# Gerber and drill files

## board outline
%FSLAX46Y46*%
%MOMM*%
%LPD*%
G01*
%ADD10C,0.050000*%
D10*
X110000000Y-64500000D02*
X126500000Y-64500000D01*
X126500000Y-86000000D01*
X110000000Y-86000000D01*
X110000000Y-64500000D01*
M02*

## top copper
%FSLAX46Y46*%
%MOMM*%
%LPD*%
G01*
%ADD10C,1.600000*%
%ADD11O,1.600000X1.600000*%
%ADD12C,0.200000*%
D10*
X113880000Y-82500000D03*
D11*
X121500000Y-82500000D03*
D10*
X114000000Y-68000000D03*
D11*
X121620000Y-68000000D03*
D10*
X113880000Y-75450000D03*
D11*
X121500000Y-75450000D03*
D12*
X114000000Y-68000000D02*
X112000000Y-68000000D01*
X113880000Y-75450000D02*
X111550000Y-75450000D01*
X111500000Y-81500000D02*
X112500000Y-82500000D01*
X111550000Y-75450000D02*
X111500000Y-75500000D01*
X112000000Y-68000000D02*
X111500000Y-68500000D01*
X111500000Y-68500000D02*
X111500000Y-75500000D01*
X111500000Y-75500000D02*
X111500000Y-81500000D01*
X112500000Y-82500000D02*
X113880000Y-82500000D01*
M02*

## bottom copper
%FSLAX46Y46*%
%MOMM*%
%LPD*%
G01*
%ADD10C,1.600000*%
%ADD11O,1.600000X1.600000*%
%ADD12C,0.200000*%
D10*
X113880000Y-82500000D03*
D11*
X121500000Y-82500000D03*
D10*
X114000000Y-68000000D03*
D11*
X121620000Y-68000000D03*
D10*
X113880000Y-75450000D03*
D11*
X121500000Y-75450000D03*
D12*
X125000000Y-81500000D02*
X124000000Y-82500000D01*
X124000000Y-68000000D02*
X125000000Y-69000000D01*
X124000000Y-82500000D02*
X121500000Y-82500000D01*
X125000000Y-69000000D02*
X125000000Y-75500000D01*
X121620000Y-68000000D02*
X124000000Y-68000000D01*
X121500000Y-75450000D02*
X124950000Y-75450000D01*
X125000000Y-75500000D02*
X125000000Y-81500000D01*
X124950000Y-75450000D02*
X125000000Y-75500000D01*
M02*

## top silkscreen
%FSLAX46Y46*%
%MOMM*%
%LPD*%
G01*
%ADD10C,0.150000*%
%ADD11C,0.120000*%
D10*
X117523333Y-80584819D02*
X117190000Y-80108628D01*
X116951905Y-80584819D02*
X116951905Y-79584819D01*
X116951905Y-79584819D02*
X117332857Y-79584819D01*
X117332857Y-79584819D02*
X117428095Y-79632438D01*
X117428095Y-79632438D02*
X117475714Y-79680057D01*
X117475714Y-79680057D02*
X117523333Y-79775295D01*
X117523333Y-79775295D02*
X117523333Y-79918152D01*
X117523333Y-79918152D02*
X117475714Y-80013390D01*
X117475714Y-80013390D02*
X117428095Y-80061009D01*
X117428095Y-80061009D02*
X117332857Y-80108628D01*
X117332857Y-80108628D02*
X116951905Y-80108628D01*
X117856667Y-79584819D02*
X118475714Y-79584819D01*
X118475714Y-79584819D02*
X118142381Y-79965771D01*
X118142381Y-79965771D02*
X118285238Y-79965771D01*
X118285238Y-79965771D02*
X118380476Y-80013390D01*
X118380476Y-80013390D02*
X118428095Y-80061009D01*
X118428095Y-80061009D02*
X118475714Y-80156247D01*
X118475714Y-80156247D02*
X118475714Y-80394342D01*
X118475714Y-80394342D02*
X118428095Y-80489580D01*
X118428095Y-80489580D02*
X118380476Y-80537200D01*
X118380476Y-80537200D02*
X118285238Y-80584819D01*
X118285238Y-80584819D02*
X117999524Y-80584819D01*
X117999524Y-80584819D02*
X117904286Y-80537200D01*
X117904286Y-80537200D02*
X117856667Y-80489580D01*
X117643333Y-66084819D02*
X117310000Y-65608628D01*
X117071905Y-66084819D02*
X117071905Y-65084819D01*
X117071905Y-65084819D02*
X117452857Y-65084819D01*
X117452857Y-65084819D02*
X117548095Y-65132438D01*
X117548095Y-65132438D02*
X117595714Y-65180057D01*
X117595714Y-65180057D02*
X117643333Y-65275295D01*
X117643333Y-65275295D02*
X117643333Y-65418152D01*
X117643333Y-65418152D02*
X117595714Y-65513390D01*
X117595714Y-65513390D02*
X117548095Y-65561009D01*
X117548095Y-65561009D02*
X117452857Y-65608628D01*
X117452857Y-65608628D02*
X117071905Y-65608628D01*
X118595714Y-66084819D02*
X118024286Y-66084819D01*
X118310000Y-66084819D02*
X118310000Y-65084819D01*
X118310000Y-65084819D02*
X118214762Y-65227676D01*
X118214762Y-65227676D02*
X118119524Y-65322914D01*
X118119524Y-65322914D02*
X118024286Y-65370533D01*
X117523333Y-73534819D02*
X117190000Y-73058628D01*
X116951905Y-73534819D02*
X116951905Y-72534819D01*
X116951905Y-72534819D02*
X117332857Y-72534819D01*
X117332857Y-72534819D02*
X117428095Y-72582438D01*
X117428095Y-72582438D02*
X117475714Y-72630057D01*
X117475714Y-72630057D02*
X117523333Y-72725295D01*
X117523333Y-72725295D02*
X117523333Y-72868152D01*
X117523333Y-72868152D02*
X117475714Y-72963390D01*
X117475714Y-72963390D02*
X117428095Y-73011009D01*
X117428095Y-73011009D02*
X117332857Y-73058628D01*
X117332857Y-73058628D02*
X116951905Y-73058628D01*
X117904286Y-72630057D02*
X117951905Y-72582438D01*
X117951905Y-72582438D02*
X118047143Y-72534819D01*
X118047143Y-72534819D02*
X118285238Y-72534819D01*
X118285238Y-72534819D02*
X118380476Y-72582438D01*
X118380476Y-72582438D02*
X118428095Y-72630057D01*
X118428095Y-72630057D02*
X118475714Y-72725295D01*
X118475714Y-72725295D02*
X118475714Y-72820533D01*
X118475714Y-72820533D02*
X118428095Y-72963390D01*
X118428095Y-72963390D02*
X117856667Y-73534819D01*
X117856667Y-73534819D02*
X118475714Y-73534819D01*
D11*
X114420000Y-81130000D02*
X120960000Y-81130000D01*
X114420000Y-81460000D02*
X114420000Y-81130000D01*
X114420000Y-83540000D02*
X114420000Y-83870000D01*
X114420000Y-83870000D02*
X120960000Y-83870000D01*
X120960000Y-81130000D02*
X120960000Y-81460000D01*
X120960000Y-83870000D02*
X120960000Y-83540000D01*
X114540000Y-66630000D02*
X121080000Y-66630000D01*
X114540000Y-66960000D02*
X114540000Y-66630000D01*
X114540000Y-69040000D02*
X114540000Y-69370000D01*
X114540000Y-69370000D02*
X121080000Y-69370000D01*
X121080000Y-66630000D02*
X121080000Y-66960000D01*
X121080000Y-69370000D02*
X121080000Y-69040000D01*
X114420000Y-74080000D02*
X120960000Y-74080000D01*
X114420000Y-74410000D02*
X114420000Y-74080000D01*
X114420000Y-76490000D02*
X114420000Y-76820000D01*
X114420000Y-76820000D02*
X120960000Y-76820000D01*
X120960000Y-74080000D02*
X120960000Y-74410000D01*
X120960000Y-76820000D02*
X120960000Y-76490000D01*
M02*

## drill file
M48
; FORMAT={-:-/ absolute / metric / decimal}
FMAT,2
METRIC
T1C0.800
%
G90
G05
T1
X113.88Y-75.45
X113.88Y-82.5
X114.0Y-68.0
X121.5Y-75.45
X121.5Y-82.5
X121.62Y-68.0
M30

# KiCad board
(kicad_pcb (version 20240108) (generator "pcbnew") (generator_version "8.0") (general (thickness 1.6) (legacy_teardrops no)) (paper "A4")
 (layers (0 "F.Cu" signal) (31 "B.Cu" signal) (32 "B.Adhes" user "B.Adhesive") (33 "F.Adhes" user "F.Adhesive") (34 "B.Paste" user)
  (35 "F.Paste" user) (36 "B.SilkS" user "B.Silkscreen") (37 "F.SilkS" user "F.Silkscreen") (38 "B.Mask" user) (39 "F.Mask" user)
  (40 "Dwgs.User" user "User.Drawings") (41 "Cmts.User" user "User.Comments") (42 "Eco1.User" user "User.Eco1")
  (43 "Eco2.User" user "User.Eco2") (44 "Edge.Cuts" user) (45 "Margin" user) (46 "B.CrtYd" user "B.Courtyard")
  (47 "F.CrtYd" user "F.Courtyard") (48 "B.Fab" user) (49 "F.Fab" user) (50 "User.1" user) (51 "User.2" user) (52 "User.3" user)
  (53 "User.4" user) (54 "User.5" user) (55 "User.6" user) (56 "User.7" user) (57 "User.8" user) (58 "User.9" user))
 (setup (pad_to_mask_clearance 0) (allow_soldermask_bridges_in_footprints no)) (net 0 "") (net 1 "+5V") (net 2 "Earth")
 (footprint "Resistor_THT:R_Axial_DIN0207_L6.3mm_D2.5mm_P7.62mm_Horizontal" (layer "F.Cu") (at 113.88 82.5)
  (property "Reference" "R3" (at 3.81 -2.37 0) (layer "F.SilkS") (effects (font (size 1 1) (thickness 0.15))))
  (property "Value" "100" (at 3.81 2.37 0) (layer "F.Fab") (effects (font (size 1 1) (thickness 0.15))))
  (fp_line (start 0.54 -1.37) (end 7.08 -1.37) (stroke (width 0.12) (type solid)) (layer "F.SilkS"))
  (fp_line (start 0.54 -1.04) (end 0.54 -1.37) (stroke (width 0.12) (type solid)) (layer "F.SilkS"))
  (fp_line (start 0.54 1.04) (end 0.54 1.37) (stroke (width 0.12) (type solid)) (layer "F.SilkS"))
  (fp_line (start 0.54 1.37) (end 7.08 1.37) (stroke (width 0.12) (type solid)) (layer "F.SilkS"))
  (fp_line (start 7.08 -1.37) (end 7.08 -1.04) (stroke (width 0.12) (type solid)) (layer "F.SilkS"))
  (fp_line (start 7.08 1.37) (end 7.08 1.04) (stroke (width 0.12) (type solid)) (layer "F.SilkS"))
  (pad "1" thru_hole circle (at 0 0) (size 1.6 1.6) (drill 0.8) (layers "*.Cu" "*.Mask") (remove_unused_layers no) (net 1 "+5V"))
  (pad "2" thru_hole oval (at 7.62 0) (size 1.6 1.6) (drill 0.8) (layers "*.Cu" "*.Mask") (remove_unused_layers no) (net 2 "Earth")))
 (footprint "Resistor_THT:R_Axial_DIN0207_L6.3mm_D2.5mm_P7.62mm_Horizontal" (layer "F.Cu") (at 114 68)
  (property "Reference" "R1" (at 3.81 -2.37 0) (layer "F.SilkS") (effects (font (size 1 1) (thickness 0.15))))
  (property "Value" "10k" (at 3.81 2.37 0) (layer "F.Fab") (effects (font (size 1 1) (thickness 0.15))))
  (fp_line (start 0.54 -1.37) (end 7.08 -1.37) (stroke (width 0.12) (type solid)) (layer "F.SilkS"))
  (fp_line (start 0.54 -1.04) (end 0.54 -1.37) (stroke (width 0.12) (type solid)) (layer "F.SilkS"))
  (fp_line (start 0.54 1.04) (end 0.54 1.37) (stroke (width 0.12) (type solid)) (layer "F.SilkS"))
  (fp_line (start 0.54 1.37) (end 7.08 1.37) (stroke (width 0.12) (type solid)) (layer "F.SilkS"))
  (fp_line (start 7.08 -1.37) (end 7.08 -1.04) (stroke (width 0.12) (type solid)) (layer "F.SilkS"))
  (fp_line (start 7.08 1.37) (end 7.08 1.04) (stroke (width 0.12) (type solid)) (layer "F.SilkS"))
  (pad "1" thru_hole circle (at 0 0) (size 1.6 1.6) (drill 0.8) (layers "*.Cu" "*.Mask") (remove_unused_layers no) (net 1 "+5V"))
  (pad "2" thru_hole oval (at 7.62 0) (size 1.6 1.6) (drill 0.8) (layers "*.Cu" "*.Mask") (remove_unused_layers no) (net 2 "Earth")))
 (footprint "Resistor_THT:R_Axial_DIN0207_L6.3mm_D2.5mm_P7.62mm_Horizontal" (layer "F.Cu") (at 113.88 75.45)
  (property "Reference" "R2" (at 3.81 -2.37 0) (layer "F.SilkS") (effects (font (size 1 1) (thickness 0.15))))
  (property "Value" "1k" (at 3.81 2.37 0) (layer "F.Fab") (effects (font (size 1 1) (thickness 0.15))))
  (fp_line (start 0.54 -1.37) (end 7.08 -1.37) (stroke (width 0.12) (type solid)) (layer "F.SilkS"))
  (fp_line (start 0.54 -1.04) (end 0.54 -1.37) (stroke (width 0.12) (type solid)) (layer "F.SilkS"))
  (fp_line (start 0.54 1.04) (end 0.54 1.37) (stroke (width 0.12) (type solid)) (layer "F.SilkS"))
  (fp_line (start 0.54 1.37) (end 7.08 1.37) (stroke (width 0.12) (type solid)) (layer "F.SilkS"))
  (fp_line (start 7.08 -1.37) (end 7.08 -1.04) (stroke (width 0.12) (type solid)) (layer "F.SilkS"))
  (fp_line (start 7.08 1.37) (end 7.08 1.04) (stroke (width 0.12) (type solid)) (layer "F.SilkS"))
  (pad "1" thru_hole circle (at 0 0) (size 1.6 1.6) (drill 0.8) (layers "*.Cu" "*.Mask") (remove_unused_layers no) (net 1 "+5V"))
  (pad "2" thru_hole oval (at 7.62 0) (size 1.6 1.6) (drill 0.8) (layers "*.Cu" "*.Mask") (remove_unused_layers no) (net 2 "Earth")))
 (gr_rect (start 110 64.5) (end 126.5 86) (stroke (width 0.05) (type default)) (fill none) (layer "Edge.Cuts"))
 (segment (start 125 81.5) (end 124 82.5) (width 0.2) (layer "B.Cu") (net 2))
 (segment (start 124 68) (end 125 69) (width 0.2) (layer "B.Cu") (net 2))
 (segment (start 124 82.5) (end 121.5 82.5) (width 0.2) (layer "B.Cu") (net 2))
 (segment (start 125 69) (end 125 75.5) (width 0.2) (layer "B.Cu") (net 2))
 (segment (start 121.62 68) (end 124 68) (width 0.2) (layer "B.Cu") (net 2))
 (segment (start 121.5 75.45) (end 124.95 75.45) (width 0.2) (layer "B.Cu") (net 2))
 (segment (start 125 75.5) (end 125 81.5) (width 0.2) (layer "B.Cu") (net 2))
 (segment (start 124.95 75.45) (end 125 75.5) (width 0.2) (layer "B.Cu") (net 2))
 (segment (start 114 68) (end 112 68) (width 0.2) (layer "F.Cu") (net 1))
 (segment (start 113.88 75.45) (end 111.55 75.45) (width 0.2) (layer "F.Cu") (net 1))
 (segment (start 111.5 81.5) (end 112.5 82.5) (width 0.2) (layer "F.Cu") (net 1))
 (segment (start 111.55 75.45) (end 111.5 75.5) (width 0.2) (layer "F.Cu") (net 1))
 (segment (start 112 68) (end 111.5 68.5) (width 0.2) (layer "F.Cu") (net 1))
 (segment (start 111.5 68.5) (end 111.5 75.5) (width 0.2) (layer "F.Cu") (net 1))
 (segment (start 111.5 75.5) (end 111.5 81.5) (width 0.2) (layer "F.Cu") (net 1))
 (segment (start 112.5 82.5) (end 113.88 82.5) (width 0.2) (layer "F.Cu") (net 1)))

